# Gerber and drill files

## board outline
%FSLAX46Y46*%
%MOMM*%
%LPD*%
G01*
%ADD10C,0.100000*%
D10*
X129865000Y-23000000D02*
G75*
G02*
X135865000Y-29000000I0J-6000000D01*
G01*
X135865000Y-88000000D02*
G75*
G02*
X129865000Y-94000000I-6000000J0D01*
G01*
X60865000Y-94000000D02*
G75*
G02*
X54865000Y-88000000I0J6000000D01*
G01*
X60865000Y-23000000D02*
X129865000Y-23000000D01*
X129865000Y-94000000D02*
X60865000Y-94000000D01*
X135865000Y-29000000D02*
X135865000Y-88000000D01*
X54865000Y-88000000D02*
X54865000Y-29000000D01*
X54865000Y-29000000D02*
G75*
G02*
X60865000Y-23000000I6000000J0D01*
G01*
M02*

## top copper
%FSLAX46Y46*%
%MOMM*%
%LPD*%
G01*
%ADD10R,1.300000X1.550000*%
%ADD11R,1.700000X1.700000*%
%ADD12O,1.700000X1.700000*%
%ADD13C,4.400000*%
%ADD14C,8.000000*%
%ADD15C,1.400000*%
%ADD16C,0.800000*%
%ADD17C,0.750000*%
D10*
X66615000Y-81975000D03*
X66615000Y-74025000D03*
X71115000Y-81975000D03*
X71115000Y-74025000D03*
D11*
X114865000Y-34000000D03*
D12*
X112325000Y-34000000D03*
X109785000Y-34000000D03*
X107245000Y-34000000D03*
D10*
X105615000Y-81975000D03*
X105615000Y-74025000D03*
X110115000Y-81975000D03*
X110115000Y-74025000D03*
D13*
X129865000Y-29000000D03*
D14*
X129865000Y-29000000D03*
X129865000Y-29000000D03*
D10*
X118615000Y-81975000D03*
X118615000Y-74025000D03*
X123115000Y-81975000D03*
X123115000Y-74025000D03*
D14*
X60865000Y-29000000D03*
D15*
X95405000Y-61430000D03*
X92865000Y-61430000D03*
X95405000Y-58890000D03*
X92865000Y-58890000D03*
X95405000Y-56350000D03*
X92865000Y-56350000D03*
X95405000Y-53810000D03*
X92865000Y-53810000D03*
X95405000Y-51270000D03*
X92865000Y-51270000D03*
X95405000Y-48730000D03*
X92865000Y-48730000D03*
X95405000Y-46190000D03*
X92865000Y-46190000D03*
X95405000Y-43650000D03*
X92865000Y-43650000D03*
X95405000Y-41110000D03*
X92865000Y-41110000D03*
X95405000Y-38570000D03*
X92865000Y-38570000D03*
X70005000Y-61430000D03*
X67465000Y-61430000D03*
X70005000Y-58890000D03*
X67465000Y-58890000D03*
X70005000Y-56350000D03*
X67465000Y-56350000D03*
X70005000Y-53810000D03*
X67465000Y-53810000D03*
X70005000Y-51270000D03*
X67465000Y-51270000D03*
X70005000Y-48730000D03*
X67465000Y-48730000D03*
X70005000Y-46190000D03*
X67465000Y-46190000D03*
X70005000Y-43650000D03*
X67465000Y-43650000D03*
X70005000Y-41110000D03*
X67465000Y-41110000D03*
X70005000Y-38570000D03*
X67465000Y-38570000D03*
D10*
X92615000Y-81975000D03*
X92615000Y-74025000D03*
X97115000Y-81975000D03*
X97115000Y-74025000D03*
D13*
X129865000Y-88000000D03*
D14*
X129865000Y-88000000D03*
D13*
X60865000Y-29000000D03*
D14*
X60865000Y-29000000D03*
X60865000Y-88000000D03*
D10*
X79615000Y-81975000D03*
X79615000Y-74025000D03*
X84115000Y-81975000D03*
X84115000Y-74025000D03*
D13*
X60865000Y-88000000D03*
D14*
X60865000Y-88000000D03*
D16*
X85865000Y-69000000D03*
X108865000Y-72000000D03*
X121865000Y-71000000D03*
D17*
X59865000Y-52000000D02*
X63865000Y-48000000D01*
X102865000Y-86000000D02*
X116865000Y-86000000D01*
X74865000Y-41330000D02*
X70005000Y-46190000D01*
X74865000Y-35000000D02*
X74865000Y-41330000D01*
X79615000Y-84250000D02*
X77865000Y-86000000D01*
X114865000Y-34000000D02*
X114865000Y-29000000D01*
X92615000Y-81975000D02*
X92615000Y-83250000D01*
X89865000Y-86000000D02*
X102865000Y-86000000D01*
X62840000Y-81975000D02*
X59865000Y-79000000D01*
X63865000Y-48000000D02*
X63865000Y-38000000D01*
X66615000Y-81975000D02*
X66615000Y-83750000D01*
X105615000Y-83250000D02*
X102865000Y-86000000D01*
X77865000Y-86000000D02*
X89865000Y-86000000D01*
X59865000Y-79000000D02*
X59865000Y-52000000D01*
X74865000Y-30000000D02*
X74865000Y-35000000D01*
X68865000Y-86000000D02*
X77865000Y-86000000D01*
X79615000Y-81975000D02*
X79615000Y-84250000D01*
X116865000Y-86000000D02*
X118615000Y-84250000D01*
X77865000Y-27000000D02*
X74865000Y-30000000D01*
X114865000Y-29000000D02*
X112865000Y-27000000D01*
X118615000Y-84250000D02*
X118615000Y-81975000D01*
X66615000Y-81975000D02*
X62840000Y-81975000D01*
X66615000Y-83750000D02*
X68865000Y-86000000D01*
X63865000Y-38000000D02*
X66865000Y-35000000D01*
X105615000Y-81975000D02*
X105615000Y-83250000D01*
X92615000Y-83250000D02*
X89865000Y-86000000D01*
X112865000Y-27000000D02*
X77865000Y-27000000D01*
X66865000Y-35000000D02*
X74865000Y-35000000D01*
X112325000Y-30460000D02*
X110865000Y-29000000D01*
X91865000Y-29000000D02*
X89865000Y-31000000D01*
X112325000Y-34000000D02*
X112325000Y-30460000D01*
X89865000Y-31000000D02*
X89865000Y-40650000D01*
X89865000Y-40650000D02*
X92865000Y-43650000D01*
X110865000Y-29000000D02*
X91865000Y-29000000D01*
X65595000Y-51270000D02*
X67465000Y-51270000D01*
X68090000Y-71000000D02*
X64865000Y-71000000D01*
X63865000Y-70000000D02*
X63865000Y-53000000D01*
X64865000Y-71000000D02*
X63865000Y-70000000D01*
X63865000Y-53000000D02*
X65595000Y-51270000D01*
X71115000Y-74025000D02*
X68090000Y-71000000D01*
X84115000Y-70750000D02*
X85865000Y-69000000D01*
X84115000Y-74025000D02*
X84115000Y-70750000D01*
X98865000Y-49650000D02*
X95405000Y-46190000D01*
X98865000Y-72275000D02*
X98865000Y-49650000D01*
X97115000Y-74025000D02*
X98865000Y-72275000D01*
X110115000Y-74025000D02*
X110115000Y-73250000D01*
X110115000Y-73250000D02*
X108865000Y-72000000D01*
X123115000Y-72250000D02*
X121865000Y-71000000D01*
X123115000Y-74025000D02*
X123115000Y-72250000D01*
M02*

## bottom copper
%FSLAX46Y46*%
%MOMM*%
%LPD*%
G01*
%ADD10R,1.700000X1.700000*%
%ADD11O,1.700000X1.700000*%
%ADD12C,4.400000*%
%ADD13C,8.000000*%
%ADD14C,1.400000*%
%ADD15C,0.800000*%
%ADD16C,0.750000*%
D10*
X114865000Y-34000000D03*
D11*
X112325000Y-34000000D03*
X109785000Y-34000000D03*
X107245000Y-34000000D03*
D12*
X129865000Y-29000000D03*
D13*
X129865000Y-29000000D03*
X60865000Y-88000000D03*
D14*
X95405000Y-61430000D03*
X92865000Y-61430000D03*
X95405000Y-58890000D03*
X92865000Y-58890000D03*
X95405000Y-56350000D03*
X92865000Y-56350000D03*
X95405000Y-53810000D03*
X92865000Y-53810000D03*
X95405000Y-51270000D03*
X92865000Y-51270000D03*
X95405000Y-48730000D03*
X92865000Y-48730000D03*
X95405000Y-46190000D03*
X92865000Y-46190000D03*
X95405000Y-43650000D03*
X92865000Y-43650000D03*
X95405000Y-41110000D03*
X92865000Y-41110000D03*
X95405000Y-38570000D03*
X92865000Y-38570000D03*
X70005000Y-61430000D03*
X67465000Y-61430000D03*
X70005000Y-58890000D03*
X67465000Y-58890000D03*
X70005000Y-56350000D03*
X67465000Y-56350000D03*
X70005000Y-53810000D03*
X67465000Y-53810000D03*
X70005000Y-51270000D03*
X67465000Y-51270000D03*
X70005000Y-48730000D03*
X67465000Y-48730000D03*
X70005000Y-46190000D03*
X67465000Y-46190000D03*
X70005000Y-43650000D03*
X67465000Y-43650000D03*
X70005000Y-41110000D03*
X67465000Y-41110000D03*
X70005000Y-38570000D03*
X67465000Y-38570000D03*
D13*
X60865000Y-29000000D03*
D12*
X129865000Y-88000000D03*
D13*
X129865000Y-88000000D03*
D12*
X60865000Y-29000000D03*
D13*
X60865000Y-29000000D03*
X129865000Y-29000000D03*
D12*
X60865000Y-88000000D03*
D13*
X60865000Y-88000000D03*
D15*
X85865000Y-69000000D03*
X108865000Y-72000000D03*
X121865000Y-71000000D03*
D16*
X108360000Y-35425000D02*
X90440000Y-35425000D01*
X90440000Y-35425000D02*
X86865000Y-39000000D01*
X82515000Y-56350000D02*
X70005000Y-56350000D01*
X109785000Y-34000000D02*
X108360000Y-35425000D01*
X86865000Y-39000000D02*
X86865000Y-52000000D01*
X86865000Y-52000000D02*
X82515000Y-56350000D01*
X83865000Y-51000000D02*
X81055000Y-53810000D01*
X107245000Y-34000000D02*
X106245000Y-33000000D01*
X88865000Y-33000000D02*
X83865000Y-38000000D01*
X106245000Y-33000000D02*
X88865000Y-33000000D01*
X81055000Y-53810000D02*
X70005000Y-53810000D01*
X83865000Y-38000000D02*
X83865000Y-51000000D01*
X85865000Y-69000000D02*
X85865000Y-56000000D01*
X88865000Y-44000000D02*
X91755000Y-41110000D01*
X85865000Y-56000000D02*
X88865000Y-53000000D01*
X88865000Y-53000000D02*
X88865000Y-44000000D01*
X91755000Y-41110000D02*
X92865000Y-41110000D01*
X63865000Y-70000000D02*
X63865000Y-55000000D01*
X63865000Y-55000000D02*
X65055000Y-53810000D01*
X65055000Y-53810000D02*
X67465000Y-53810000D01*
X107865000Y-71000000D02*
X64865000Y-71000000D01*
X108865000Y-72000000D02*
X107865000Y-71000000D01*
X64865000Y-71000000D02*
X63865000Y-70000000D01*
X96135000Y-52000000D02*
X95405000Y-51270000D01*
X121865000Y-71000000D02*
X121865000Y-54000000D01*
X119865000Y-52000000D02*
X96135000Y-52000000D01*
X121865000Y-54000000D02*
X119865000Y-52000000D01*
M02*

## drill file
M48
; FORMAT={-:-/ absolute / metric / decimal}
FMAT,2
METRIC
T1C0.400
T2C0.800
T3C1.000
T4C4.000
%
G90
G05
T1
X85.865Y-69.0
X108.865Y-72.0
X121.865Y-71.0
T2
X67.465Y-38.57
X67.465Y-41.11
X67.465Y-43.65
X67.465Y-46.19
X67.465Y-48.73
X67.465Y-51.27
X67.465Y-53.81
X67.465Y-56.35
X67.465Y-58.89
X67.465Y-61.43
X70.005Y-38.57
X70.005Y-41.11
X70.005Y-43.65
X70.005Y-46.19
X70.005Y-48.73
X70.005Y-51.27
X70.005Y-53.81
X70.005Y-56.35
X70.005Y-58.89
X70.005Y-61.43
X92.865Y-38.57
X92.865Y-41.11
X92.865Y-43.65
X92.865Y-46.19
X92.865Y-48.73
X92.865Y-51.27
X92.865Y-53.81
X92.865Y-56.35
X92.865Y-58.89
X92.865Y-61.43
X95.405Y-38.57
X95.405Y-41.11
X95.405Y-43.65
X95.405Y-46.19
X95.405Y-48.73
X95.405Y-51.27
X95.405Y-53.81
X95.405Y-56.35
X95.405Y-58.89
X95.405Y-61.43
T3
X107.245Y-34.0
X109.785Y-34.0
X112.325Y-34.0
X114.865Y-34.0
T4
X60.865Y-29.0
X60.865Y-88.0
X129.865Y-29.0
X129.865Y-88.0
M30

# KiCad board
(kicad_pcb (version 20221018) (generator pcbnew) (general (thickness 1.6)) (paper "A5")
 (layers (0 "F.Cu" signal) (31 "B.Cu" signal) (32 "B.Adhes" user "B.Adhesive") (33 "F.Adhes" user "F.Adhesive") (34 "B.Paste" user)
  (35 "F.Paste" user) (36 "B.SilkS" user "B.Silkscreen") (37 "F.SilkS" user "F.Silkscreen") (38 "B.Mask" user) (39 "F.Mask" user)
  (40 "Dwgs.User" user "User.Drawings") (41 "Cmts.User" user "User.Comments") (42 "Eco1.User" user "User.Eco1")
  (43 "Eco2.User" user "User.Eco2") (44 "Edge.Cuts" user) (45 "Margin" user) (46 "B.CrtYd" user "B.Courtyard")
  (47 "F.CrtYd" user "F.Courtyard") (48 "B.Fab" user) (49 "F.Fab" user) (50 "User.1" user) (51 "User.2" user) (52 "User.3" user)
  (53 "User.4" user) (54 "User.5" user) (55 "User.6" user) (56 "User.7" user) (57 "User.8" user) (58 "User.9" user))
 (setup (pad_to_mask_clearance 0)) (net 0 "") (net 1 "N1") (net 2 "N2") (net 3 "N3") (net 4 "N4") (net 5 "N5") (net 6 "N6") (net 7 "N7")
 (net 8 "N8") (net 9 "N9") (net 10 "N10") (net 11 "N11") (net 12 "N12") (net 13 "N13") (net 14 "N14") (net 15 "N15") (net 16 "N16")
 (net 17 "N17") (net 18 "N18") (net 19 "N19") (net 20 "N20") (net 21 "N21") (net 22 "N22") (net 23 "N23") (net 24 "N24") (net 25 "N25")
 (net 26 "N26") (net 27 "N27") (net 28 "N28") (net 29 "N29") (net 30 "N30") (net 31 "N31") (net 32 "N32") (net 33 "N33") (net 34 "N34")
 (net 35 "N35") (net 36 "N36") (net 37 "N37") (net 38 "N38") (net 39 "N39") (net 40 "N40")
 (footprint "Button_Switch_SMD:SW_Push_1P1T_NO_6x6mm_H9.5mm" (layer "F.Cu") (at 68.865 78 90)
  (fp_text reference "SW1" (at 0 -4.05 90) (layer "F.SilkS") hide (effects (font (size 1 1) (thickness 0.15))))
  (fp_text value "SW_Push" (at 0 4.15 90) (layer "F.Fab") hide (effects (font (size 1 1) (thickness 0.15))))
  (pad "1" smd rect (at -3.975 -2.25 90) (size 1.55 1.3) (layers "F.Cu" "F.Paste" "F.Mask") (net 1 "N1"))
  (pad "1" smd rect (at 3.975 -2.25 90) (size 1.55 1.3) (layers "F.Cu" "F.Paste" "F.Mask") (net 1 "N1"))
  (pad "2" smd rect (at -3.975 2.25 90) (size 1.55 1.3) (layers "F.Cu" "F.Paste" "F.Mask") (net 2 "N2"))
  (pad "2" smd rect (at 3.975 2.25 90) (size 1.55 1.3) (layers "F.Cu" "F.Paste" "F.Mask") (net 2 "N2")))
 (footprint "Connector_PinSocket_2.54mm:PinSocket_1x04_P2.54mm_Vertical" (layer "F.Cu") (at 114.865 34 -90)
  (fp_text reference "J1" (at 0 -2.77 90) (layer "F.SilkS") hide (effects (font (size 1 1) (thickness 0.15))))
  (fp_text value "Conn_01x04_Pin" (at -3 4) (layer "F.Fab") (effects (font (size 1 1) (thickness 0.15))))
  (pad "1" thru_hole rect (at 0 0 270) (size 1.7 1.7) (drill 1) (layers "*.Cu" "*.Mask") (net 1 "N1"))
  (pad "2" thru_hole oval (at 0 2.54 270) (size 1.7 1.7) (drill 1) (layers "*.Cu" "*.Mask") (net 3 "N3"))
  (pad "3" thru_hole oval (at 0 5.08 270) (size 1.7 1.7) (drill 1) (layers "*.Cu" "*.Mask") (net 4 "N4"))
  (pad "4" thru_hole oval (at 0 7.62 270) (size 1.7 1.7) (drill 1) (layers "*.Cu" "*.Mask") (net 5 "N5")))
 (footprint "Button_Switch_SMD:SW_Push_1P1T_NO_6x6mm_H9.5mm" (layer "F.Cu") (at 107.865 78 90)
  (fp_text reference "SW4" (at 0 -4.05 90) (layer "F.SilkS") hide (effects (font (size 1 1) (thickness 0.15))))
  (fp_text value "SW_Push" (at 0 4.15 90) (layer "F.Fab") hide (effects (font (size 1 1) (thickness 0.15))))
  (pad "1" smd rect (at -3.975 -2.25 90) (size 1.55 1.3) (layers "F.Cu" "F.Paste" "F.Mask") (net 1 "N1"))
  (pad "1" smd rect (at 3.975 -2.25 90) (size 1.55 1.3) (layers "F.Cu" "F.Paste" "F.Mask") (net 1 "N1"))
  (pad "2" smd rect (at -3.975 2.25 90) (size 1.55 1.3) (layers "F.Cu" "F.Paste" "F.Mask") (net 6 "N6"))
  (pad "2" smd rect (at 3.975 2.25 90) (size 1.55 1.3) (layers "F.Cu" "F.Paste" "F.Mask") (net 6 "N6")))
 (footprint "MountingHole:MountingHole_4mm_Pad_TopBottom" (layer "F.Cu") (at 129.865 29)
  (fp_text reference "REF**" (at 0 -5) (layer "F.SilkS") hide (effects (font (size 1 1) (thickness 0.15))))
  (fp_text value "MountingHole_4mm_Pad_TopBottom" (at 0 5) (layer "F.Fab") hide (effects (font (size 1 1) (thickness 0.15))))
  (pad "1" thru_hole circle (at 0 0) (size 4.4 4.4) (drill 4) (layers "*.Cu" "*.Mask"))
  (pad "1" connect circle (at 0 0) (size 8 8) (layers "F.Cu" "F.Mask"))
  (pad "1" connect circle (at 0 0) (size 8 8) (layers "B.Cu" "B.Mask")))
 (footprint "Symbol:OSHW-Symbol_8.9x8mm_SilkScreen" (layer "F.Cu") (at 105.365 64)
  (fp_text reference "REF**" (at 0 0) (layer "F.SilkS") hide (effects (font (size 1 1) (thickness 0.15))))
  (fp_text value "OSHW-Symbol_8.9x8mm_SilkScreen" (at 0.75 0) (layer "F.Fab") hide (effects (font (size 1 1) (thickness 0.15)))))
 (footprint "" (layer "F.Cu") (at 60.865 88)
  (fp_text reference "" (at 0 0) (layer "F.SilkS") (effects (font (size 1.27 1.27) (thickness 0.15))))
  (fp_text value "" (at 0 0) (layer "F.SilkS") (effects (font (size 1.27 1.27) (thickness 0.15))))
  (pad "1" connect circle (at 0 0) (size 8 8) (layers "B.Cu" "B.Mask")))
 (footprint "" (layer "F.Cu") (at 129.865 29)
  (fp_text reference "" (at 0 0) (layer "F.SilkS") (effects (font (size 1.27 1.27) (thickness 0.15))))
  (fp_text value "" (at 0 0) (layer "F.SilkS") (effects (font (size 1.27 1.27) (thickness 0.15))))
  (pad "1" connect circle (at 0 0) (size 8 8) (layers "F.Cu" "F.Mask")))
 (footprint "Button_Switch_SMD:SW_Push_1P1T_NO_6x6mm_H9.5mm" (layer "F.Cu") (at 120.865 78 90)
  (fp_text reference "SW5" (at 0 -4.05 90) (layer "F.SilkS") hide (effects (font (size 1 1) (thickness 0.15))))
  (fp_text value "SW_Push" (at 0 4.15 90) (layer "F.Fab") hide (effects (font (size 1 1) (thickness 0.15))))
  (pad "1" smd rect (at -3.975 -2.25 90) (size 1.55 1.3) (layers "F.Cu" "F.Paste" "F.Mask") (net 1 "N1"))
  (pad "1" smd rect (at 3.975 -2.25 90) (size 1.55 1.3) (layers "F.Cu" "F.Paste" "F.Mask") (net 1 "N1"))
  (pad "2" smd rect (at -3.975 2.25 90) (size 1.55 1.3) (layers "F.Cu" "F.Paste" "F.Mask") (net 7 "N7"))
  (pad "2" smd rect (at 3.975 2.25 90) (size 1.55 1.3) (layers "F.Cu" "F.Paste" "F.Mask") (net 7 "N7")))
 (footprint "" (layer "F.Cu") (at 60.865 29)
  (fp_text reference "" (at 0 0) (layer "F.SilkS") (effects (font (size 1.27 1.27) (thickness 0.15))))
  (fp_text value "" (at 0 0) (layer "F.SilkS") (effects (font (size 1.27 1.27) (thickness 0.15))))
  (pad "1" connect circle (at 0 0) (size 8 8) (layers "F.Cu" "F.Mask")))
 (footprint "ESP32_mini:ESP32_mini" (layer "F.Cu") (at 81.435 50 180)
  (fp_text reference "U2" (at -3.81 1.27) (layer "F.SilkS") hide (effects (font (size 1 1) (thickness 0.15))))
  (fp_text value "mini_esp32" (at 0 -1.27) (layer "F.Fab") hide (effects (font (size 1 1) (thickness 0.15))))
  (pad "1" thru_hole circle (at -13.97 -11.43 90) (size 1.4 1.4) (drill 0.8) (layers "*.Cu" "*.Mask") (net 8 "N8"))
  (pad "2" thru_hole circle (at -11.43 -11.43 90) (size 1.4 1.4) (drill 0.8) (layers "*.Cu" "*.Mask") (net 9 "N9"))
  (pad "3" thru_hole circle (at -13.97 -8.89 90) (size 1.4 1.4) (drill 0.8) (layers "*.Cu" "*.Mask") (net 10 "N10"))
  (pad "4" thru_hole circle (at -11.43 -8.89 90) (size 1.4 1.4) (drill 0.8) (layers "*.Cu" "*.Mask") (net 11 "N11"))
  (pad "5" thru_hole circle (at -13.97 -6.35 90) (size 1.4 1.4) (drill 0.8) (layers "*.Cu" "*.Mask") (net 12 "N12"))
  (pad "6" thru_hole circle (at -11.43 -6.35 90) (size 1.4 1.4) (drill 0.8) (layers "*.Cu" "*.Mask") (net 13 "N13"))
  (pad "7" thru_hole circle (at -13.97 -3.81 90) (size 1.4 1.4) (drill 0.8) (layers "*.Cu" "*.Mask") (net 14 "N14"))
  (pad "8" thru_hole circle (at -11.43 -3.81 90) (size 1.4 1.4) (drill 0.8) (layers "*.Cu" "*.Mask") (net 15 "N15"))
  (pad "9" thru_hole circle (at -13.97 -1.27 90) (size 1.4 1.4) (drill 0.8) (layers "*.Cu" "*.Mask") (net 7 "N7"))
  (pad "10" thru_hole circle (at -11.43 -1.27 90) (size 1.4 1.4) (drill 0.8) (layers "*.Cu" "*.Mask") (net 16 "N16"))
  (pad "11" thru_hole circle (at -13.97 1.27 90) (size 1.4 1.4) (drill 0.8) (layers "*.Cu" "*.Mask") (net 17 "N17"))
  (pad "12" thru_hole circle (at -11.43 1.27 90) (size 1.4 1.4) (drill 0.8) (layers "*.Cu" "*.Mask") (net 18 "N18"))
  (pad "13" thru_hole circle (at -13.97 3.81 90) (size 1.4 1.4) (drill 0.8) (layers "*.Cu" "*.Mask") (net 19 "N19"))
  (pad "14" thru_hole circle (at -11.43 3.81 90) (size 1.4 1.4) (drill 0.8) (layers "*.Cu" "*.Mask") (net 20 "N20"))
  (pad "15" thru_hole circle (at -13.97 6.35 90) (size 1.4 1.4) (drill 0.8) (layers "*.Cu" "*.Mask") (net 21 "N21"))
  (pad "16" thru_hole circle (at -11.43 6.35 90) (size 1.4 1.4) (drill 0.8) (layers "*.Cu" "*.Mask") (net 3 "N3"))
  (pad "17" thru_hole circle (at -13.97 8.89 90) (size 1.4 1.4) (drill 0.8) (layers "*.Cu" "*.Mask") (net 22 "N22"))
  (pad "18" thru_hole circle (at -11.43 8.89 90) (size 1.4 1.4) (drill 0.8) (layers "*.Cu" "*.Mask") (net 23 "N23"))
  (pad "19" thru_hole circle (at -13.97 11.43 90) (size 1.4 1.4) (drill 0.8) (layers "*.Cu" "*.Mask") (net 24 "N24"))
  (pad "20" thru_hole circle (at -11.43 11.43 90) (size 1.4 1.4) (drill 0.8) (layers "*.Cu" "*.Mask") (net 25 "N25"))
  (pad "21" thru_hole circle (at 11.43 -11.43 90) (size 1.4 1.4) (drill 0.8) (layers "*.Cu" "*.Mask") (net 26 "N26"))
  (pad "22" thru_hole circle (at 13.97 -11.43 90) (size 1.4 1.4) (drill 0.8) (layers "*.Cu" "*.Mask") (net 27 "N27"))
  (pad "23" thru_hole circle (at 11.43 -8.89 90) (size 1.4 1.4) (drill 0.8) (layers "*.Cu" "*.Mask") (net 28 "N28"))
  (pad "24" thru_hole circle (at 13.97 -8.89 90) (size 1.4 1.4) (drill 0.8) (layers "*.Cu" "*.Mask") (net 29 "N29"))
  (pad "25" thru_hole circle (at 11.43 -6.35 90) (size 1.4 1.4) (drill 0.8) (layers "*.Cu" "*.Mask") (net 4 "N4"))
  (pad "26" thru_hole circle (at 13.97 -6.35 90) (size 1.4 1.4) (drill 0.8) (layers "*.Cu" "*.Mask") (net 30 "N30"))
  (pad "27" thru_hole circle (at 11.43 -3.81 90) (size 1.4 1.4) (drill 0.8) (layers "*.Cu" "*.Mask") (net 5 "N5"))
  (pad "28" thru_hole circle (at 13.97 -3.81 90) (size 1.4 1.4) (drill 0.8) (layers "*.Cu" "*.Mask") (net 6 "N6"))
  (pad "29" thru_hole circle (at 11.43 -1.27 90) (size 1.4 1.4) (drill 0.8) (layers "*.Cu" "*.Mask") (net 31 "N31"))
  (pad "30" thru_hole circle (at 13.97 -1.27 90) (size 1.4 1.4) (drill 0.8) (layers "*.Cu" "*.Mask") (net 2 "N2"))
  (pad "31" thru_hole circle (at 11.43 1.27 90) (size 1.4 1.4) (drill 0.8) (layers "*.Cu" "*.Mask") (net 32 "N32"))
  (pad "32" thru_hole circle (at 13.97 1.27 90) (size 1.4 1.4) (drill 0.8) (layers "*.Cu" "*.Mask") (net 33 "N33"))
  (pad "33" thru_hole circle (at 11.43 3.81 90) (size 1.4 1.4) (drill 0.8) (layers "*.Cu" "*.Mask") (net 1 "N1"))
  (pad "34" thru_hole circle (at 13.97 3.81 90) (size 1.4 1.4) (drill 0.8) (layers "*.Cu" "*.Mask") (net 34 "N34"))
  (pad "35" thru_hole circle (at 11.43 6.35 90) (size 1.4 1.4) (drill 0.8) (layers "*.Cu" "*.Mask") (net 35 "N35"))
  (pad "36" thru_hole circle (at 13.97 6.35 90) (size 1.4 1.4) (drill 0.8) (layers "*.Cu" "*.Mask") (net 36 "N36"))
  (pad "37" thru_hole circle (at 11.43 8.89 90) (size 1.4 1.4) (drill 0.8) (layers "*.Cu" "*.Mask") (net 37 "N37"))
  (pad "38" thru_hole circle (at 13.97 8.89 90) (size 1.4 1.4) (drill 0.8) (layers "*.Cu" "*.Mask") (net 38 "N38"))
  (pad "39" thru_hole circle (at 11.43 11.43 90) (size 1.4 1.4) (drill 0.8) (layers "*.Cu" "*.Mask") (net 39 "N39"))
  (pad "40" thru_hole circle (at 13.97 11.43 90) (size 1.4 1.4) (drill 0.8) (layers "*.Cu" "*.Mask") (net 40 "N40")))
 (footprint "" (layer "F.Cu") (at 60.865 29)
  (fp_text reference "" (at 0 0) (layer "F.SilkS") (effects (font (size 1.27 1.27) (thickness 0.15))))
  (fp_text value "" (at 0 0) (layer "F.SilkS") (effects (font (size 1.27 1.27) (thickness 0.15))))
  (pad "1" connect circle (at 0 0) (size 8 8) (layers "B.Cu" "B.Mask")))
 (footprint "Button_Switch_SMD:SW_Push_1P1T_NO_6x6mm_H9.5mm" (layer "F.Cu") (at 94.865 78 90)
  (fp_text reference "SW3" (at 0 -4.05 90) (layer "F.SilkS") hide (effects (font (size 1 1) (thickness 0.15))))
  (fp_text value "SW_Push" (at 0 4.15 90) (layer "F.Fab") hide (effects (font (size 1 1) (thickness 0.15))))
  (pad "1" smd rect (at -3.975 -2.25 90) (size 1.55 1.3) (layers "F.Cu" "F.Paste" "F.Mask") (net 1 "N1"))
  (pad "1" smd rect (at 3.975 -2.25 90) (size 1.55 1.3) (layers "F.Cu" "F.Paste" "F.Mask") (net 1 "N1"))
  (pad "2" smd rect (at -3.975 2.25 90) (size 1.55 1.3) (layers "F.Cu" "F.Paste" "F.Mask") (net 19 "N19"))
  (pad "2" smd rect (at 3.975 2.25 90) (size 1.55 1.3) (layers "F.Cu" "F.Paste" "F.Mask") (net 19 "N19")))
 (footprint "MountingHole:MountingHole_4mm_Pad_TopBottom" (layer "F.Cu") (at 129.865 88)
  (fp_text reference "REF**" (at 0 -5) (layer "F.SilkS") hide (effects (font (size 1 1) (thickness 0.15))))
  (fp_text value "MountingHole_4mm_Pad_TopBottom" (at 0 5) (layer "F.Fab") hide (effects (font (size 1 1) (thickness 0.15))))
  (pad "1" thru_hole circle (at 0 0) (size 4.4 4.4) (drill 4) (layers "*.Cu" "*.Mask"))
  (pad "1" connect circle (at 0 0) (size 8 8) (layers "F.Cu" "F.Mask"))
  (pad "1" connect circle (at 0 0) (size 8 8) (layers "B.Cu" "B.Mask")))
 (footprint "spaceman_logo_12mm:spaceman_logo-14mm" (layer "F.Cu") (at 116.365 63.5)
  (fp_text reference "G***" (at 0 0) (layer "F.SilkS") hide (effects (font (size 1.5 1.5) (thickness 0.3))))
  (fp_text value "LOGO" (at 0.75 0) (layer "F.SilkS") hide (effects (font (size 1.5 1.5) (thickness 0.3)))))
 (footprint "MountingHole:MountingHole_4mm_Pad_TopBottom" (layer "F.Cu") (at 60.865 29)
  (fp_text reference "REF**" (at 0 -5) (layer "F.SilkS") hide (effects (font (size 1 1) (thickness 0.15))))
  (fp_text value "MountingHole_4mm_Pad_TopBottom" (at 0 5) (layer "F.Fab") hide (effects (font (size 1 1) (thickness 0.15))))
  (pad "1" thru_hole circle (at 0 0) (size 4.4 4.4) (drill 4) (layers "*.Cu" "*.Mask"))
  (pad "1" connect circle (at 0 0) (size 8 8) (layers "F.Cu" "F.Mask"))
  (pad "1" connect circle (at 0 0) (size 8 8) (layers "B.Cu" "B.Mask")))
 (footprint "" (layer "F.Cu") (at 60.865 88)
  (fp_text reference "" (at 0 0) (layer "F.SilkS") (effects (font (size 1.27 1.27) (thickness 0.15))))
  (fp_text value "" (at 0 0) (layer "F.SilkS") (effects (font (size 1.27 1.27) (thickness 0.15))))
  (pad "1" connect circle (at 0 0) (size 8 8) (layers "F.Cu" "F.Mask")))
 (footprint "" (layer "F.Cu") (at 129.865 29)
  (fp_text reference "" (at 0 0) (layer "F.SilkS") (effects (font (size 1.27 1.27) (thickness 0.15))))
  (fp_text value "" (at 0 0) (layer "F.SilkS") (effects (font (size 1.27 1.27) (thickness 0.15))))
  (pad "1" connect circle (at 0 0) (size 8 8) (layers "B.Cu" "B.Mask")))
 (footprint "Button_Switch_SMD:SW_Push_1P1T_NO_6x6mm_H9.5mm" (layer "F.Cu") (at 81.865 78 90)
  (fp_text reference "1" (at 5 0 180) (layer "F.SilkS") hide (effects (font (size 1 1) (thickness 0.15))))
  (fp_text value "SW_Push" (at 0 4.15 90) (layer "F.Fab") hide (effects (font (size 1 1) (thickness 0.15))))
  (pad "1" smd rect (at -3.975 -2.25 90) (size 1.55 1.3) (layers "F.Cu" "F.Paste" "F.Mask") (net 1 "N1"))
  (pad "1" smd rect (at 3.975 -2.25 90) (size 1.55 1.3) (layers "F.Cu" "F.Paste" "F.Mask") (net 1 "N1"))
  (pad "2" smd rect (at -3.975 2.25 90) (size 1.55 1.3) (layers "F.Cu" "F.Paste" "F.Mask") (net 23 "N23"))
  (pad "2" smd rect (at 3.975 2.25 90) (size 1.55 1.3) (layers "F.Cu" "F.Paste" "F.Mask") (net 23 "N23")))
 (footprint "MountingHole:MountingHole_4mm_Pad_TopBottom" (layer "F.Cu") (at 60.865 88)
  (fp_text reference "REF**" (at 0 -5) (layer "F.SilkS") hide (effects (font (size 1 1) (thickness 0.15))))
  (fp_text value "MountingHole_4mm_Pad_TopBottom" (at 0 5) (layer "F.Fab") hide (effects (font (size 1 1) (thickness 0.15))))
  (pad "1" thru_hole circle (at 0 0) (size 4.4 4.4) (drill 4) (layers "*.Cu" "*.Mask"))
  (pad "1" connect circle (at 0 0) (size 8 8) (layers "F.Cu" "F.Mask"))
  (pad "1" connect circle (at 0 0) (size 8 8) (layers "B.Cu" "B.Mask")))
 (gr_arc (start 129.865 23) (mid 134.107641 24.757359) (end 135.865 29) (stroke (width 0.1) (type default)) (layer "Edge.Cuts"))
 (gr_arc (start 135.865 88) (mid 134.107641 92.242641) (end 129.865 94) (stroke (width 0.1) (type default)) (layer "Edge.Cuts"))
 (gr_arc (start 60.865 94) (mid 56.622359 92.242641) (end 54.865 88) (stroke (width 0.1) (type default)) (layer "Edge.Cuts"))
 (gr_line (start 60.865 23) (end 129.865 23) (stroke (width 0.1) (type default)) (layer "Edge.Cuts"))
 (gr_line (start 129.865 94) (end 60.865 94) (stroke (width 0.1) (type default)) (layer "Edge.Cuts"))
 (gr_line (start 135.865 29) (end 135.865 88) (stroke (width 0.1) (type default)) (layer "Edge.Cuts"))
 (gr_line (start 54.865 88) (end 54.865 29) (stroke (width 0.1) (type default)) (layer "Edge.Cuts"))
 (gr_arc (start 54.865 29) (mid 56.622359 24.757359) (end 60.865 23) (stroke (width 0.1) (type default)) (layer "Edge.Cuts"))
 (segment (start 59.865 52) (end 63.865 48) (width 0.75) (layer "F.Cu") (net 1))
 (segment (start 102.865 86) (end 116.865 86) (width 0.75) (layer "F.Cu") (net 1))
 (segment (start 74.865 41.33) (end 70.005 46.19) (width 0.75) (layer "F.Cu") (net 1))
 (segment (start 74.865 35) (end 74.865 41.33) (width 0.75) (layer "F.Cu") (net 1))
 (segment (start 79.615 84.25) (end 77.865 86) (width 0.75) (layer "F.Cu") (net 1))
 (segment (start 114.865 34) (end 114.865 29) (width 0.75) (layer "F.Cu") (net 1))
 (segment (start 92.615 81.975) (end 92.615 83.25) (width 0.75) (layer "F.Cu") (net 1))
 (segment (start 89.865 86) (end 102.865 86) (width 0.75) (layer "F.Cu") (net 1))
 (segment (start 62.84 81.975) (end 59.865 79) (width 0.75) (layer "F.Cu") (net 1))
 (segment (start 63.865 48) (end 63.865 38) (width 0.75) (layer "F.Cu") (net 1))
 (segment (start 66.615 81.975) (end 66.615 83.75) (width 0.75) (layer "F.Cu") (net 1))
 (segment (start 105.615 83.25) (end 102.865 86) (width 0.75) (layer "F.Cu") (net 1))
 (segment (start 77.865 86) (end 89.865 86) (width 0.75) (layer "F.Cu") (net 1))
 (segment (start 59.865 79) (end 59.865 52) (width 0.75) (layer "F.Cu") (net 1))
 (segment (start 74.865 30) (end 74.865 35) (width 0.75) (layer "F.Cu") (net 1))
 (segment (start 68.865 86) (end 77.865 86) (width 0.75) (layer "F.Cu") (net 1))
 (segment (start 79.615 81.975) (end 79.615 84.25) (width 0.75) (layer "F.Cu") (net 1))
 (segment (start 116.865 86) (end 118.615 84.25) (width 0.75) (layer "F.Cu") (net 1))
 (segment (start 77.865 27) (end 74.865 30) (width 0.75) (layer "F.Cu") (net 1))
 (segment (start 114.865 29) (end 112.865 27) (width 0.75) (layer "F.Cu") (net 1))
 (segment (start 118.615 84.25) (end 118.615 81.975) (width 0.75) (layer "F.Cu") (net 1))
 (segment (start 66.615 81.975) (end 62.84 81.975) (width 0.75) (layer "F.Cu") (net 1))
 (segment (start 66.615 83.75) (end 68.865 86) (width 0.75) (layer "F.Cu") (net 1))
 (segment (start 63.865 38) (end 66.865 35) (width 0.75) (layer "F.Cu") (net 1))
 (segment (start 105.615 81.975) (end 105.615 83.25) (width 0.75) (layer "F.Cu") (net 1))
 (segment (start 92.615 83.25) (end 89.865 86) (width 0.75) (layer "F.Cu") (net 1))
 (segment (start 112.865 27) (end 77.865 27) (width 0.75) (layer "F.Cu") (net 1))
 (segment (start 66.865 35) (end 74.865 35) (width 0.75) (layer "F.Cu") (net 1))
 (segment (start 112.325 30.46) (end 110.865 29) (width 0.75) (layer "F.Cu") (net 3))
 (segment (start 91.865 29) (end 89.865 31) (width 0.75) (layer "F.Cu") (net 3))
 (segment (start 112.325 34) (end 112.325 30.46) (width 0.75) (layer "F.Cu") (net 3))
 (segment (start 89.865 31) (end 89.865 40.65) (width 0.75) (layer "F.Cu") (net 3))
 (segment (start 89.865 40.65) (end 92.865 43.65) (width 0.75) (layer "F.Cu") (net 3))
 (segment (start 110.865 29) (end 91.865 29) (width 0.75) (layer "F.Cu") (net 3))
 (segment (start 108.36 35.425) (end 90.44 35.425) (width 0.75) (layer "B.Cu") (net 4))
 (segment (start 90.44 35.425) (end 86.865 39) (width 0.75) (layer "B.Cu") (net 4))
 (segment (start 82.515 56.35) (end 70.005 56.35) (width 0.75) (layer "B.Cu") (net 4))
 (segment (start 109.785 34) (end 108.36 35.425) (width 0.75) (layer "B.Cu") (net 4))
 (segment (start 86.865 39) (end 86.865 52) (width 0.75) (layer "B.Cu") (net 4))
 (segment (start 86.865 52) (end 82.515 56.35) (width 0.75) (layer "B.Cu") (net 4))
 (segment (start 83.865 51) (end 81.055 53.81) (width 0.75) (layer "B.Cu") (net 5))
 (segment (start 107.245 34) (end 106.245 33) (width 0.75) (layer "B.Cu") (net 5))
 (segment (start 88.865 33) (end 83.865 38) (width 0.75) (layer "B.Cu") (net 5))
 (segment (start 106.245 33) (end 88.865 33) (width 0.75) (layer "B.Cu") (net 5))
 (segment (start 81.055 53.81) (end 70.005 53.81) (width 0.75) (layer "B.Cu") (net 5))
 (segment (start 83.865 38) (end 83.865 51) (width 0.75) (layer "B.Cu") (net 5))
 (segment (start 65.595 51.27) (end 67.465 51.27) (width 0.75) (layer "F.Cu") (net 2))
 (segment (start 68.09 71) (end 64.865 71) (width 0.75) (layer "F.Cu") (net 2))
 (segment (start 63.865 70) (end 63.865 53) (width 0.75) (layer "F.Cu") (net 2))
 (segment (start 64.865 71) (end 63.865 70) (width 0.75) (layer "F.Cu") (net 2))
 (segment (start 63.865 53) (end 65.595 51.27) (width 0.75) (layer "F.Cu") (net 2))
 (segment (start 71.115 74.025) (end 68.09 71) (width 0.75) (layer "F.Cu") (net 2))
 (segment (start 84.115 70.75) (end 85.865 69) (width 0.75) (layer "F.Cu") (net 23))
 (segment (start 84.115 74.025) (end 84.115 70.75) (width 0.75) (layer "F.Cu") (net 23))
 (via (at 85.865 69) (size 0.8) (drill 0.4) (layers "F.Cu" "B.Cu") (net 23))
 (segment (start 85.865 69) (end 85.865 56) (width 0.75) (layer "B.Cu") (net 23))
 (segment (start 88.865 44) (end 91.755 41.11) (width 0.75) (layer "B.Cu") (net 23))
 (segment (start 85.865 56) (end 88.865 53) (width 0.75) (layer "B.Cu") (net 23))
 (segment (start 88.865 53) (end 88.865 44) (width 0.75) (layer "B.Cu") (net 23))
 (segment (start 91.755 41.11) (end 92.865 41.11) (width 0.75) (layer "B.Cu") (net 23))
 (segment (start 98.865 49.65) (end 95.405 46.19) (width 0.75) (layer "F.Cu") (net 19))
 (segment (start 98.865 72.275) (end 98.865 49.65) (width 0.75) (layer "F.Cu") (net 19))
 (segment (start 97.115 74.025) (end 98.865 72.275) (width 0.75) (layer "F.Cu") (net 19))
 (segment (start 110.115 74.025) (end 110.115 73.25) (width 0.75) (layer "F.Cu") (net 6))
 (segment (start 110.115 73.25) (end 108.865 72) (width 0.75) (layer "F.Cu") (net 6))
 (via (at 108.865 72) (size 0.8) (drill 0.4) (layers "F.Cu" "B.Cu") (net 6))
 (segment (start 63.865 70) (end 63.865 55) (width 0.75) (layer "B.Cu") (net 6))
 (segment (start 63.865 55) (end 65.055 53.81) (width 0.75) (layer "B.Cu") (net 6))
 (segment (start 65.055 53.81) (end 67.465 53.81) (width 0.75) (layer "B.Cu") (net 6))
 (segment (start 107.865 71) (end 64.865 71) (width 0.75) (layer "B.Cu") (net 6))
 (segment (start 108.865 72) (end 107.865 71) (width 0.75) (layer "B.Cu") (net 6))
 (segment (start 64.865 71) (end 63.865 70) (width 0.75) (layer "B.Cu") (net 6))
 (segment (start 123.115 72.25) (end 121.865 71) (width 0.75) (layer "F.Cu") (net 7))
 (segment (start 123.115 74.025) (end 123.115 72.25) (width 0.75) (layer "F.Cu") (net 7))
 (via (at 121.865 71) (size 0.8) (drill 0.4) (layers "F.Cu" "B.Cu") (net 7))
 (segment (start 96.135 52) (end 95.405 51.27) (width 0.75) (layer "B.Cu") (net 7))
 (segment (start 121.865 71) (end 121.865 54) (width 0.75) (layer "B.Cu") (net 7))
 (segment (start 119.865 52) (end 96.135 52) (width 0.75) (layer "B.Cu") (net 7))
 (segment (start 121.865 54) (end 119.865 52) (width 0.75) (layer "B.Cu") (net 7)))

